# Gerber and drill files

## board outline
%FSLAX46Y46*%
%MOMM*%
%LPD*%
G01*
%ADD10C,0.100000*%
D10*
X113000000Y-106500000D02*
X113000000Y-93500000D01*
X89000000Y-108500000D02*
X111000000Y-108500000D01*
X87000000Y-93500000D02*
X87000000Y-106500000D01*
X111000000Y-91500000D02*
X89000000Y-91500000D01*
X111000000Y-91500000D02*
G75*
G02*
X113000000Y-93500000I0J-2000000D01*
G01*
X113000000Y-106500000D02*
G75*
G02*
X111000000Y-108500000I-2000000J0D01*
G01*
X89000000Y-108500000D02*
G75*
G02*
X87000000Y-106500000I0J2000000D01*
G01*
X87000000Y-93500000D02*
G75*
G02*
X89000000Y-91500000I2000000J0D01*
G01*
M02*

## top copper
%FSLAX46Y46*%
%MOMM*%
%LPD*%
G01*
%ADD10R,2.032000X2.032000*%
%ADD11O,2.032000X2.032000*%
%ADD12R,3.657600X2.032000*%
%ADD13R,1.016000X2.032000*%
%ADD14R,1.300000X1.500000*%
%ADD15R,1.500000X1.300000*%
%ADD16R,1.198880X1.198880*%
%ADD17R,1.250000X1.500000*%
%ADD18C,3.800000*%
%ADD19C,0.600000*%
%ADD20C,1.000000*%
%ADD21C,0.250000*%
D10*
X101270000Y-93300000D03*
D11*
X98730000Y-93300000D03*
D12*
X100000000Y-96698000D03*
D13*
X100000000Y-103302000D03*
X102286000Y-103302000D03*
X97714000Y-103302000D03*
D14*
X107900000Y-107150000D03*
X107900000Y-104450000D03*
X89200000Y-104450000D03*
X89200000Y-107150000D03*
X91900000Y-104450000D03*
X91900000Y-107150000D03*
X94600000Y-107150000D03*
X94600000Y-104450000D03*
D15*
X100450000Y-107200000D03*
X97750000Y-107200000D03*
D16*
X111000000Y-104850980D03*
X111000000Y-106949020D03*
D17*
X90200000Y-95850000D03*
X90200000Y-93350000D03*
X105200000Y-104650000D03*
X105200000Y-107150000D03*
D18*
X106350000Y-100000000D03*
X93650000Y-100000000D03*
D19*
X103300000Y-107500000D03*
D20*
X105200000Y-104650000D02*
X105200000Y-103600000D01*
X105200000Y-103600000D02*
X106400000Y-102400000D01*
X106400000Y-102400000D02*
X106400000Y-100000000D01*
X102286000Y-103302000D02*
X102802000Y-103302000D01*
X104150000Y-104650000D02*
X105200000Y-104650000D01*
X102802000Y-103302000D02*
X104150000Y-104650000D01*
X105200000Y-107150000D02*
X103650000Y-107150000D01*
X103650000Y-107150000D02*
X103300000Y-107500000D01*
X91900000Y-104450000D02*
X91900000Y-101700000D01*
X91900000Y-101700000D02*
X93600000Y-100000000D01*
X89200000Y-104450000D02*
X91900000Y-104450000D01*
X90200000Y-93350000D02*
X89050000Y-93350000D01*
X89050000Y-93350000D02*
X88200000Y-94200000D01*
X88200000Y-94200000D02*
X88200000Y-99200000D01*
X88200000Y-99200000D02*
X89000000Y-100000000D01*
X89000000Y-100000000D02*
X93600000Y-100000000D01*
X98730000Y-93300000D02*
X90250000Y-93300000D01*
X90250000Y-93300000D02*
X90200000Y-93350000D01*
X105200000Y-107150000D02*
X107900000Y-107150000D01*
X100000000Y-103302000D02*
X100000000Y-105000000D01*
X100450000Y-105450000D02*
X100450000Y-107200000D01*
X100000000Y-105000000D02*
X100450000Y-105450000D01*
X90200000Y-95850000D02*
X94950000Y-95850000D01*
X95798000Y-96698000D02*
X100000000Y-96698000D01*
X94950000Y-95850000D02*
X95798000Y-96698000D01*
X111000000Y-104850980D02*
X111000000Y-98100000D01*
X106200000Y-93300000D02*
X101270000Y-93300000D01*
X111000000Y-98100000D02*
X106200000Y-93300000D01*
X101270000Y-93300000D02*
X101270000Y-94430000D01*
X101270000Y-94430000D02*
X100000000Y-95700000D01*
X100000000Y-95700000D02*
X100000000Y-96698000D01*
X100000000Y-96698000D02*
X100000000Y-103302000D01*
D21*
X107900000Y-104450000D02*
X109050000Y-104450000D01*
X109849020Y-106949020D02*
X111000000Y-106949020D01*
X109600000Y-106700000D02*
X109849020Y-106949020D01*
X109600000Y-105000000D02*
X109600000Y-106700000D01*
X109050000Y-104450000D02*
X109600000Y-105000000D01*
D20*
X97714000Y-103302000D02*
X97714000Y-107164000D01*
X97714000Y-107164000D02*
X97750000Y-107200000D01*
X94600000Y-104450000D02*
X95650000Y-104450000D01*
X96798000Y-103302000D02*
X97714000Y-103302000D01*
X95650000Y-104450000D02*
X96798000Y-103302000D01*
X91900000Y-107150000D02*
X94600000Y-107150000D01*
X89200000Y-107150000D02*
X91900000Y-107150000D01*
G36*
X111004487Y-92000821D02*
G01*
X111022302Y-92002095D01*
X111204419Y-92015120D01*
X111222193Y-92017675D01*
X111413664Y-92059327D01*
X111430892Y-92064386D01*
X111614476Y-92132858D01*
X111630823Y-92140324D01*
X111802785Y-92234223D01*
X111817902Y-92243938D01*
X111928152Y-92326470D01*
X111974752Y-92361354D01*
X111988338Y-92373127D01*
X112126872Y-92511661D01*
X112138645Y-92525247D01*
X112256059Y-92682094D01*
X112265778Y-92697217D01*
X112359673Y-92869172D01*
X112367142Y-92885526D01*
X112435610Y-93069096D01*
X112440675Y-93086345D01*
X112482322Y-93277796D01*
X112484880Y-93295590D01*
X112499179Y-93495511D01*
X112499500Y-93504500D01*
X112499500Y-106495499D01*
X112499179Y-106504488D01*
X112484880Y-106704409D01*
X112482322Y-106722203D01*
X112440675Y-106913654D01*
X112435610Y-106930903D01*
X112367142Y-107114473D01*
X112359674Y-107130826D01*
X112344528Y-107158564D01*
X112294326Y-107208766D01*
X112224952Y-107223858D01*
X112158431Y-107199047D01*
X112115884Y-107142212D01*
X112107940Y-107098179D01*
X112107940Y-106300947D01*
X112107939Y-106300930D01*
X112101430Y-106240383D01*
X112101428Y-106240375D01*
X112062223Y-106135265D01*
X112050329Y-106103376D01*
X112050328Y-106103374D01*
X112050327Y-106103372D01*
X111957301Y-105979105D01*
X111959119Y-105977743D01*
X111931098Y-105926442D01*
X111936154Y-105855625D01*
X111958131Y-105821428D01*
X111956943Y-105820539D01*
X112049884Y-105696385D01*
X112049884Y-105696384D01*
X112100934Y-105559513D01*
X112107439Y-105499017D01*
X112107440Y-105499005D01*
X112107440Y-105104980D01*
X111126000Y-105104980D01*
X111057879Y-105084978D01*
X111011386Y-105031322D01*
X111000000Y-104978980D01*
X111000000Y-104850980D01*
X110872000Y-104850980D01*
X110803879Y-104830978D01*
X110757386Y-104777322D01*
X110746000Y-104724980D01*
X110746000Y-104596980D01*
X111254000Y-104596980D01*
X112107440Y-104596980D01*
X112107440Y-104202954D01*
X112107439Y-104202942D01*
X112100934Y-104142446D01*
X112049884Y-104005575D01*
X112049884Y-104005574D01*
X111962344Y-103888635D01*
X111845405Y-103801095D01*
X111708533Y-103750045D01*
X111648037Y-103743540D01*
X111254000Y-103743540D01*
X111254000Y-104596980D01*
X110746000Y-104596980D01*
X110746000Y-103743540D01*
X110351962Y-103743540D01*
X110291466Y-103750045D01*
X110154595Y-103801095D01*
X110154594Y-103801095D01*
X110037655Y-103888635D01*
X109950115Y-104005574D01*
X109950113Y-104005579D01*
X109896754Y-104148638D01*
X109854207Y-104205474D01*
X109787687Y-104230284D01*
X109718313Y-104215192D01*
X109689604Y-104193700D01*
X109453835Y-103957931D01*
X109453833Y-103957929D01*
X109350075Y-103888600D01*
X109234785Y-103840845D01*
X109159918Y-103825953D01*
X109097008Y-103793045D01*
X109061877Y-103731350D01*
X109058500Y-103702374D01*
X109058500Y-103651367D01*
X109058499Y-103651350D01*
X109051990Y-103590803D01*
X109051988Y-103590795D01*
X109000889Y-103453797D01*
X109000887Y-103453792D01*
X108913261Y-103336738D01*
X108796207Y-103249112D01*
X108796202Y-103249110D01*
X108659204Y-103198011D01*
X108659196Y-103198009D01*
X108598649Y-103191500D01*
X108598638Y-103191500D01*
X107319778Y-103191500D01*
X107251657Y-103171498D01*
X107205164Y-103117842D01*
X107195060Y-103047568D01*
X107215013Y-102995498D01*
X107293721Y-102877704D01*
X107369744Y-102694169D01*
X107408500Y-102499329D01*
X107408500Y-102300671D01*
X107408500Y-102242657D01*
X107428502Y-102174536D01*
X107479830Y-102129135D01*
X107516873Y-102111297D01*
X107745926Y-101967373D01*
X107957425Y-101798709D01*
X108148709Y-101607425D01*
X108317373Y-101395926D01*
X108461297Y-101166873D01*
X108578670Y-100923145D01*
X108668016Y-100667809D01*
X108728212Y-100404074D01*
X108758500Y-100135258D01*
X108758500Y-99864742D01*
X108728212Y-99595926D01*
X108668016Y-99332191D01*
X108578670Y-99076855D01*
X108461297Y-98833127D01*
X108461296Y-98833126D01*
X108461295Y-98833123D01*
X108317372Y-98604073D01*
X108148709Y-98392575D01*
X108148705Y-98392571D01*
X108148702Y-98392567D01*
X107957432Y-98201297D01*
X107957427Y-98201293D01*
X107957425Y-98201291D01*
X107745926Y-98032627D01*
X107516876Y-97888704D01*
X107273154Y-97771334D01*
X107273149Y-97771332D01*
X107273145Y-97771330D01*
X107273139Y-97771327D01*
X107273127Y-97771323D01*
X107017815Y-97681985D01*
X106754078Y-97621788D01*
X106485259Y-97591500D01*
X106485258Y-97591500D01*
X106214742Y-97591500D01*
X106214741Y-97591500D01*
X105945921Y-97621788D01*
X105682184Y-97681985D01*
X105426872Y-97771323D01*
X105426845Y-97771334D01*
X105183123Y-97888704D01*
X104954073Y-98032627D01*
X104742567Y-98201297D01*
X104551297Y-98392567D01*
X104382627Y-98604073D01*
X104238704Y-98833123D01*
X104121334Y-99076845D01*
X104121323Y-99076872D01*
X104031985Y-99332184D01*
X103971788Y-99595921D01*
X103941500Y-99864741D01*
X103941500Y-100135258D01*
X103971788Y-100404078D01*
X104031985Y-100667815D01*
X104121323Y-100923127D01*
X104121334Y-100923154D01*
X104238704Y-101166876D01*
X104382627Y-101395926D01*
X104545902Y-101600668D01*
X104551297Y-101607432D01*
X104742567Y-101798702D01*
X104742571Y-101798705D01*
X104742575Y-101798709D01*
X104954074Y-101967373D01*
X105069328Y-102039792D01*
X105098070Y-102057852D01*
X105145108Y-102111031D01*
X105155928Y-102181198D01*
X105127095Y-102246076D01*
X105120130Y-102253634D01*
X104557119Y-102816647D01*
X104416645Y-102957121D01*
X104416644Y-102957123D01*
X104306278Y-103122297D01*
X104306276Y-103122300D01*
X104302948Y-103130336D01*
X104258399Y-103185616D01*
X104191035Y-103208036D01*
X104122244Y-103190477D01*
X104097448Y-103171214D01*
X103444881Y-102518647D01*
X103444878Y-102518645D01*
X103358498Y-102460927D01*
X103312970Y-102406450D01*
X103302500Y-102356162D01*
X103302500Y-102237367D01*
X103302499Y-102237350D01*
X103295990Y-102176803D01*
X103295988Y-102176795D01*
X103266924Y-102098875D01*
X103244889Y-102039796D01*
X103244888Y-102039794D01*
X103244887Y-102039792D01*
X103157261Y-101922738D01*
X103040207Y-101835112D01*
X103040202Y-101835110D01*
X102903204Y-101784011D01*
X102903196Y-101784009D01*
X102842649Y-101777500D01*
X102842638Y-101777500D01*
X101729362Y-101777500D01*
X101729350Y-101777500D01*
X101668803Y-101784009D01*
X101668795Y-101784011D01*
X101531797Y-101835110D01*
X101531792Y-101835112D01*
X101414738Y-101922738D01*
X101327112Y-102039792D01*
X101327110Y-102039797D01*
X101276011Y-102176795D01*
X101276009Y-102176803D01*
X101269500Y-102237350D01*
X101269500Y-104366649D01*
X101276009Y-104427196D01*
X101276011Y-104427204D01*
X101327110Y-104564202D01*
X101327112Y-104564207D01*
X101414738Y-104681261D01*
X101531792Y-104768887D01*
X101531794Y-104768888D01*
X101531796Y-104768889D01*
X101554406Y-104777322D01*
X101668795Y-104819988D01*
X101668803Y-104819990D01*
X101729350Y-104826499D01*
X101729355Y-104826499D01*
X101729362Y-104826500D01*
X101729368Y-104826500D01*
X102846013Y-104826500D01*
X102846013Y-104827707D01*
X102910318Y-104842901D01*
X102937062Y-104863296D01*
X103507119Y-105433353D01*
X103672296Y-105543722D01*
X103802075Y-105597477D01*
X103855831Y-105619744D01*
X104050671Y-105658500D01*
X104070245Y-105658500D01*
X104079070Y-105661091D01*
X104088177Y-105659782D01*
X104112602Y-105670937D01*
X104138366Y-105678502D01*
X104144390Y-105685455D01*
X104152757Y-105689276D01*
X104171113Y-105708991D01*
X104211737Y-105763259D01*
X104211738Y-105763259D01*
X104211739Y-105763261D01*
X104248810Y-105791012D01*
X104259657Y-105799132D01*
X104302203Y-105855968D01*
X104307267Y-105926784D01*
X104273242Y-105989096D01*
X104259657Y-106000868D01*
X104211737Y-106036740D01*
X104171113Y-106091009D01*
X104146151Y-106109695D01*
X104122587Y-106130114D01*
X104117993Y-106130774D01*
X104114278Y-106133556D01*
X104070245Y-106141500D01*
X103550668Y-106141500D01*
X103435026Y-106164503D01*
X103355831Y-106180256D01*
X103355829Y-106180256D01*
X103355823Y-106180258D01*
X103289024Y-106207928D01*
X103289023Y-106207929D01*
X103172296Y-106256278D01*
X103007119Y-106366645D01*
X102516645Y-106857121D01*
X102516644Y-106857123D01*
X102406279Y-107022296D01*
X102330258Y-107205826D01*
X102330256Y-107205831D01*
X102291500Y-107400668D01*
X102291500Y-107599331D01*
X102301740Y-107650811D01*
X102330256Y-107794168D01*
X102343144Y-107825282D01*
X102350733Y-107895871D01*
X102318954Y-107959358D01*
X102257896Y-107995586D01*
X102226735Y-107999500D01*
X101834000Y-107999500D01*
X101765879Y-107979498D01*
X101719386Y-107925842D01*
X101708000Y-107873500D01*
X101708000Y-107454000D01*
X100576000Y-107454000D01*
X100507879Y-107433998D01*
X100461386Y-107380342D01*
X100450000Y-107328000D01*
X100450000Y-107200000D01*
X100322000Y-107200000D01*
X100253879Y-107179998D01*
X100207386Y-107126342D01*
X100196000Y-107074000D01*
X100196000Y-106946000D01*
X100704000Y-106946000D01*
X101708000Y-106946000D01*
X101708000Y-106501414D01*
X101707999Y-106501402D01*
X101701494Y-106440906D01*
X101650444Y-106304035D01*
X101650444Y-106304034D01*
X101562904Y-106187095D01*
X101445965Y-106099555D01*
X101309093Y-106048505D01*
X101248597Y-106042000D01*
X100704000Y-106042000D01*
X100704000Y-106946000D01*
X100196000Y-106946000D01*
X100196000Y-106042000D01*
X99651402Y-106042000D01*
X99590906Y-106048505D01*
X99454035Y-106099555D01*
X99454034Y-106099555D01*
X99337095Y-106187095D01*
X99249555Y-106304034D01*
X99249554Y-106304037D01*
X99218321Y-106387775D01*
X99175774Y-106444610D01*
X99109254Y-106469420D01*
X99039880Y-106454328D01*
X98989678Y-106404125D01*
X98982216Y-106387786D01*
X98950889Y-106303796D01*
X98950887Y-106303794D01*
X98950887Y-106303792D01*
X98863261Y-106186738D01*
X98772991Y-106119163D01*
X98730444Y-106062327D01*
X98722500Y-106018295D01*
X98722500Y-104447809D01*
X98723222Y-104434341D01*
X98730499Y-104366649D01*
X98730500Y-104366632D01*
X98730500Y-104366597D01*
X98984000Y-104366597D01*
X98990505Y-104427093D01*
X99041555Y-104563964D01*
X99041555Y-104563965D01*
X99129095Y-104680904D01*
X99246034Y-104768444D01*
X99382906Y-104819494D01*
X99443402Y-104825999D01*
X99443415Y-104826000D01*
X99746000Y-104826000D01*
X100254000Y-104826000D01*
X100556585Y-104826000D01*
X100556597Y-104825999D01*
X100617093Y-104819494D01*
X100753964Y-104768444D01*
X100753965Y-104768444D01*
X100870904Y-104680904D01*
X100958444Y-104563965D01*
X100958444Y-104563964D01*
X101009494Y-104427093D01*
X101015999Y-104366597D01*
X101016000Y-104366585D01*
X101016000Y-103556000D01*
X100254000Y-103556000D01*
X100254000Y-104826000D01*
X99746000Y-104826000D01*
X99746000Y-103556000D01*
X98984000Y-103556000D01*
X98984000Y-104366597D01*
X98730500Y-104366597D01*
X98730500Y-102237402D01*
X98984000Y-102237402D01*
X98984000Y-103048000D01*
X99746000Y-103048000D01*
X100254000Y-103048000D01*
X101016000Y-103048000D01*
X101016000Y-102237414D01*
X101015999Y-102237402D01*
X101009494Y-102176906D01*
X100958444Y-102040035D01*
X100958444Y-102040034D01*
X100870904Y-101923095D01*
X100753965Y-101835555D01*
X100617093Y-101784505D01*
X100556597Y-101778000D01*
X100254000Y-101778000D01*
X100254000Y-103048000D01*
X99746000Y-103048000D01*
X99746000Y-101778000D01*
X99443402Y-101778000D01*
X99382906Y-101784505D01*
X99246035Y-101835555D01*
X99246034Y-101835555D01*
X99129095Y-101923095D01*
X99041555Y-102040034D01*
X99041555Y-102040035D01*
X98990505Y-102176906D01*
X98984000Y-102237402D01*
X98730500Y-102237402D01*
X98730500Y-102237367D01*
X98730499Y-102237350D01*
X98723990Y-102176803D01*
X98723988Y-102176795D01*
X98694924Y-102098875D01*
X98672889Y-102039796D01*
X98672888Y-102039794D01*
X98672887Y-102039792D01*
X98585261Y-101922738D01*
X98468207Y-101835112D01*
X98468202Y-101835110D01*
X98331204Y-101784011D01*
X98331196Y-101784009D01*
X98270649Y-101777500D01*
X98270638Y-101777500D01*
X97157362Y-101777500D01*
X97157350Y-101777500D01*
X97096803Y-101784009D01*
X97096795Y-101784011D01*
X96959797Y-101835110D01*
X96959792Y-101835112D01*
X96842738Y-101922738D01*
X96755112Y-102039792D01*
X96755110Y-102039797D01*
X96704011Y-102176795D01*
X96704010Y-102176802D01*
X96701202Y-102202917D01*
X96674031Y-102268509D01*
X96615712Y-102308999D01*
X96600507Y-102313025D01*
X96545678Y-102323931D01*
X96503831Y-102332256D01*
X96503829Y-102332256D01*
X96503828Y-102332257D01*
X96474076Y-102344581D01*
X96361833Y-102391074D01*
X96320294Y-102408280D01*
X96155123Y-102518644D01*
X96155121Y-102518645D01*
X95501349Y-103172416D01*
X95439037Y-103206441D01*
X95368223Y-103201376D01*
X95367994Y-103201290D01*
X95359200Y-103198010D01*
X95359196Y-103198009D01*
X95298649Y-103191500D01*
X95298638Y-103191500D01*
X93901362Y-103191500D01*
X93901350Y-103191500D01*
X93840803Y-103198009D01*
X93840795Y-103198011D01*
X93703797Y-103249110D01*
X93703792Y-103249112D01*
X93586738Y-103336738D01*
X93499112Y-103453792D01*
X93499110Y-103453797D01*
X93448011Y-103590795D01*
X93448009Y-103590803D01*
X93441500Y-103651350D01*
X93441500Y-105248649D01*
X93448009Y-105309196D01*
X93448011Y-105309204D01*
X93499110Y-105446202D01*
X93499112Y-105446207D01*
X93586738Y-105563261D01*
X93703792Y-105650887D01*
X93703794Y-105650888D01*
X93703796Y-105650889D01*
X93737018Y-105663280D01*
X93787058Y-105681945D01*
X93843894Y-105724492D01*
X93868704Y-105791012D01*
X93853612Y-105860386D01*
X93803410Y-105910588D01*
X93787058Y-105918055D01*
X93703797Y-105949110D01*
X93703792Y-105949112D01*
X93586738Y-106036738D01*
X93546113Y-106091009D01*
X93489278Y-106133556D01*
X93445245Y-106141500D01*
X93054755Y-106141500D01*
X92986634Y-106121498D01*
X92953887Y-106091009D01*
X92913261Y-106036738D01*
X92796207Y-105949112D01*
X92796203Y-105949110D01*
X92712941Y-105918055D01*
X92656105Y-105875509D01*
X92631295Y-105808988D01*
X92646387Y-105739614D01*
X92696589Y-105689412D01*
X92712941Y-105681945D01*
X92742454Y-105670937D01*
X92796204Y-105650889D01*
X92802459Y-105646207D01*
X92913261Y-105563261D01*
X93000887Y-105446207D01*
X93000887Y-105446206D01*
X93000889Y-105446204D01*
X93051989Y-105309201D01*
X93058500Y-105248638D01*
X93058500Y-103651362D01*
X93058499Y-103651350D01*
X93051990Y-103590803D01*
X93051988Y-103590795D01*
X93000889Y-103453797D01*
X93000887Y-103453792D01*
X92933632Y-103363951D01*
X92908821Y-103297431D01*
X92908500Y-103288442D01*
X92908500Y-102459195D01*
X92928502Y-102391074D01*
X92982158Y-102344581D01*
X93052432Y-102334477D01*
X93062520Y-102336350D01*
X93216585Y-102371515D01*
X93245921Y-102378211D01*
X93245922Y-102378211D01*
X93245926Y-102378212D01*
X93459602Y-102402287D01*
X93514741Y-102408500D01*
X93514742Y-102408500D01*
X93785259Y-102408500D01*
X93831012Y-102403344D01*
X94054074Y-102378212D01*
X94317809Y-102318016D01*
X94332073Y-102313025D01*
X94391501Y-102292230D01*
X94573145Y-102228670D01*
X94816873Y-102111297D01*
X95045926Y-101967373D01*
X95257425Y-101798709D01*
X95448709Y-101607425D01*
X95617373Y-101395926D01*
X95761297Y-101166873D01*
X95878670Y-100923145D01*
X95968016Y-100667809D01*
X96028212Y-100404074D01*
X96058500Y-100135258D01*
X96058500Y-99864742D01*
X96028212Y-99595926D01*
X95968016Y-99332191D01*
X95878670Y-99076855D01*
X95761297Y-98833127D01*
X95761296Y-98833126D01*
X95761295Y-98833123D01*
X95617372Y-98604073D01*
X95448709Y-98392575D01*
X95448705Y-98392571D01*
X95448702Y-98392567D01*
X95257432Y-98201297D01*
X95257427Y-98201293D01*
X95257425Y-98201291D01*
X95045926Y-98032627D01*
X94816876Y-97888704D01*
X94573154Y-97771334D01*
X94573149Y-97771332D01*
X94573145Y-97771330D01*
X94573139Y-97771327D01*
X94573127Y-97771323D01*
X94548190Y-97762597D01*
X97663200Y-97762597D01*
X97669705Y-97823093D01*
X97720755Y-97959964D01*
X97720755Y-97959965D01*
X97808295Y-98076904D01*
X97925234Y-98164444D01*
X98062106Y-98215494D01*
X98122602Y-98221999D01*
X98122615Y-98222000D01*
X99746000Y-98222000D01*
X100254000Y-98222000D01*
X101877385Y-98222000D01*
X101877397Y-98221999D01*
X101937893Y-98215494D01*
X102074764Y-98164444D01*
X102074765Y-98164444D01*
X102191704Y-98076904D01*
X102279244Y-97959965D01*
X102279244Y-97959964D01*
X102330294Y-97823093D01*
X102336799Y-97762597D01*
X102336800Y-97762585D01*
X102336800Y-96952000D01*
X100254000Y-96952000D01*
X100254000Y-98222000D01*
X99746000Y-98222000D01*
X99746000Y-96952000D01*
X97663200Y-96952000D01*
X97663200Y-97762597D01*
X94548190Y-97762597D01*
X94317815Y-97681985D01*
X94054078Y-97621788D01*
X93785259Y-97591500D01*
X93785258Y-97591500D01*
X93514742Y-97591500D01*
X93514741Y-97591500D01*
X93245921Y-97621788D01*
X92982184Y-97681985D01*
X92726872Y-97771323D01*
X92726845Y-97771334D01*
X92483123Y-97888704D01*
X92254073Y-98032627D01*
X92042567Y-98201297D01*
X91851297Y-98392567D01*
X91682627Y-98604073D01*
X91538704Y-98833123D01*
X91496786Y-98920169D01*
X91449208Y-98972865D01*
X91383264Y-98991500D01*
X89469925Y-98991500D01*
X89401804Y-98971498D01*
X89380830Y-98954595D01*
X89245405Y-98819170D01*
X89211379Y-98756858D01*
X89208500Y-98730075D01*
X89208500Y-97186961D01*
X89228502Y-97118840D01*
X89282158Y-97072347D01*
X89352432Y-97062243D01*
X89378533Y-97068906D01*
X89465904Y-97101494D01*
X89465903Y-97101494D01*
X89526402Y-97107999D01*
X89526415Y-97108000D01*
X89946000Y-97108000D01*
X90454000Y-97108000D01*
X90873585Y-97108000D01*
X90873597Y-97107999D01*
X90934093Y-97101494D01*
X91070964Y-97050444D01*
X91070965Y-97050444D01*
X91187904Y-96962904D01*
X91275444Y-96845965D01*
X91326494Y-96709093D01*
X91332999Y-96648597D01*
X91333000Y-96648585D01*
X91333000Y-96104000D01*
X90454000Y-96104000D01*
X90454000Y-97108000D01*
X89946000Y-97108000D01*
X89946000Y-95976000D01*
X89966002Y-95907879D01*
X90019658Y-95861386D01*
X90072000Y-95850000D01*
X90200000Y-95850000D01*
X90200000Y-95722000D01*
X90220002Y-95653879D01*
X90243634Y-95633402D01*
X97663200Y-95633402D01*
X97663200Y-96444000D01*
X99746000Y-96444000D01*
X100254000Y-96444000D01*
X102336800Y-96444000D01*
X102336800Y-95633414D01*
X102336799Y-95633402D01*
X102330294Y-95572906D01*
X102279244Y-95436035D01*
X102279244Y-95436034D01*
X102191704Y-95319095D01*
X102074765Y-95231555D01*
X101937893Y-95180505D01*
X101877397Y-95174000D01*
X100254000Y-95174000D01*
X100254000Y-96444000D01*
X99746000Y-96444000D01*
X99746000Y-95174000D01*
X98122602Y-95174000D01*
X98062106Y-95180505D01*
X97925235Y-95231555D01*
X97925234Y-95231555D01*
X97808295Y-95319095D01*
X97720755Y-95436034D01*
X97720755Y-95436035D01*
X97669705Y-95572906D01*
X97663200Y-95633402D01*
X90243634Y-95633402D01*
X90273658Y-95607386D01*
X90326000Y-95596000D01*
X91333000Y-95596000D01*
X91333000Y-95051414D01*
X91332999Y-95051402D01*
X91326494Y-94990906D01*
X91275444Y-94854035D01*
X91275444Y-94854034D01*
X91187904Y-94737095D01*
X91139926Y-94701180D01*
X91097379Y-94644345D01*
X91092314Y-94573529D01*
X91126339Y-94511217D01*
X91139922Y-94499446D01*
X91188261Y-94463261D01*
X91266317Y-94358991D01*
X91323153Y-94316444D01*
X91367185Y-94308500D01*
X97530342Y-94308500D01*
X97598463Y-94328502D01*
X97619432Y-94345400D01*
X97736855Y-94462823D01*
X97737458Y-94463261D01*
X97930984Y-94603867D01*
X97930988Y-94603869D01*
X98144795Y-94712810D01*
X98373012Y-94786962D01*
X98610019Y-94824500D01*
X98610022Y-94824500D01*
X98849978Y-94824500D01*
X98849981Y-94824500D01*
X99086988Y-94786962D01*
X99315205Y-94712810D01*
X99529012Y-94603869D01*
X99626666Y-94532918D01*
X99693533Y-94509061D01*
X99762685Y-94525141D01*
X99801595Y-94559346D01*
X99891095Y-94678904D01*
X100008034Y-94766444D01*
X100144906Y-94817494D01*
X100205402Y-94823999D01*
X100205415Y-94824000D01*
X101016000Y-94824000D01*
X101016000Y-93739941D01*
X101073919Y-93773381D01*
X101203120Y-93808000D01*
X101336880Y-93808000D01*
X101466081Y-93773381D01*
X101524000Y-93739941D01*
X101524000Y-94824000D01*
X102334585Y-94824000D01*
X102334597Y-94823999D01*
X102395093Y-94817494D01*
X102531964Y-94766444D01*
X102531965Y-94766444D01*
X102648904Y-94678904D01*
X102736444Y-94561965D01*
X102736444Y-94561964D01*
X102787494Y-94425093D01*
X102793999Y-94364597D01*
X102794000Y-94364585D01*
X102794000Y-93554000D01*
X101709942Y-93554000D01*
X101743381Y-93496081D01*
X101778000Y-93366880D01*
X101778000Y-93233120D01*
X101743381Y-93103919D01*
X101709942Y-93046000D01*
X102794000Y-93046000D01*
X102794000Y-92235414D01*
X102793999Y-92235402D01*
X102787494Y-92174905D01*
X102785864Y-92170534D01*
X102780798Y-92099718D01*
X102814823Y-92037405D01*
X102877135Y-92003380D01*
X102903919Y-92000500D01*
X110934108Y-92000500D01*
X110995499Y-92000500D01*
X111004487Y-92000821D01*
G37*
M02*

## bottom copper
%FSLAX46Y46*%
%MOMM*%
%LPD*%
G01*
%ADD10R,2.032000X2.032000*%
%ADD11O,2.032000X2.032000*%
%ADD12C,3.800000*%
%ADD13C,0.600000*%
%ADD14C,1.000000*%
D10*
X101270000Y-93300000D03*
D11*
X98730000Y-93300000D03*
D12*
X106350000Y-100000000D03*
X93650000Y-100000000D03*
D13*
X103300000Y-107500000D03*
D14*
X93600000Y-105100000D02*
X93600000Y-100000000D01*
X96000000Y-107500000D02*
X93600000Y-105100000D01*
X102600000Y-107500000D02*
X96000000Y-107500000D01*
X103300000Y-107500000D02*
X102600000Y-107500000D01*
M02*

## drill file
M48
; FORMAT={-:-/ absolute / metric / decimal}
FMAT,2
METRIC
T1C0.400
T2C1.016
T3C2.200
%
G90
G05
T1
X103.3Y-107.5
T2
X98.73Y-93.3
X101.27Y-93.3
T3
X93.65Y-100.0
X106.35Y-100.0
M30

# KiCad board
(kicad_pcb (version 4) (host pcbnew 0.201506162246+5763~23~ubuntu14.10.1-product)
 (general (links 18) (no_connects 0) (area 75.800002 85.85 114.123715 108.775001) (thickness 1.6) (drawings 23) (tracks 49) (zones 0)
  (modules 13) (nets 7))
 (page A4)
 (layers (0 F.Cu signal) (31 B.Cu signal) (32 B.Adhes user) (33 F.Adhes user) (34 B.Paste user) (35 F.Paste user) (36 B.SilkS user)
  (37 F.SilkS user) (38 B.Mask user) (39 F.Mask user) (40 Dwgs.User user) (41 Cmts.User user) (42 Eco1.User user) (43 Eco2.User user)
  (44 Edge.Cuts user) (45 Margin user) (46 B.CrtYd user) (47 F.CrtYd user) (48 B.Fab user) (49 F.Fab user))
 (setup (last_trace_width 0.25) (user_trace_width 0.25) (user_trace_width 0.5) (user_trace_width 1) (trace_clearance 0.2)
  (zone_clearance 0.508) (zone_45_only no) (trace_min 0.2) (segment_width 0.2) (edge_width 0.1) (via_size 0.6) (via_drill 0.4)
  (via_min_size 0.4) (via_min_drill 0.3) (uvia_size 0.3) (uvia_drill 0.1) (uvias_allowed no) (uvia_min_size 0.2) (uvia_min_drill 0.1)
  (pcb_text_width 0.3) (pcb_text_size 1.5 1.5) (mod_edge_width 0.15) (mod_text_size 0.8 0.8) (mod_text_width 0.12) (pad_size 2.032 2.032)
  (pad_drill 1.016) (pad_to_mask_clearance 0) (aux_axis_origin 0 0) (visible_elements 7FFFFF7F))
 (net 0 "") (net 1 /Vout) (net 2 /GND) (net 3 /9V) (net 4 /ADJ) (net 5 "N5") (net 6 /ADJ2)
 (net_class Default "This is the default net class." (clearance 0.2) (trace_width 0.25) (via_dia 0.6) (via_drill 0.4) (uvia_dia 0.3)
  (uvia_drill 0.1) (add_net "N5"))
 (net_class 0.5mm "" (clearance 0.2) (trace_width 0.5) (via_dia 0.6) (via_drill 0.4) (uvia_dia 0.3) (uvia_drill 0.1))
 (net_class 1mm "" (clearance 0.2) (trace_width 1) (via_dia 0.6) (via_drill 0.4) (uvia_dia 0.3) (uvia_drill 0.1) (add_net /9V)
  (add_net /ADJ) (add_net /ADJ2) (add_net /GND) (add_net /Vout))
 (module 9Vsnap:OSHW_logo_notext (layer B.Cu) (at 100 102.5 180)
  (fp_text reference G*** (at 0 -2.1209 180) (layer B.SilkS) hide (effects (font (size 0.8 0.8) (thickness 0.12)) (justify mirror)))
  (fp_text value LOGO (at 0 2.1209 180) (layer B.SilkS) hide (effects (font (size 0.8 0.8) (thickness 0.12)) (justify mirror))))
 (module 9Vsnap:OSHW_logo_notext (layer F.Cu) (at 110.6 93.8)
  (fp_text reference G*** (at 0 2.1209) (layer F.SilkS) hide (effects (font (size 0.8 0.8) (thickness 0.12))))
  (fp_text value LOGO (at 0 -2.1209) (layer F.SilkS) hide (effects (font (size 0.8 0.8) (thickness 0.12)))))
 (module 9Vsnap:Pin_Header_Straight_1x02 (layer F.Cu) (at 100 93.3 270)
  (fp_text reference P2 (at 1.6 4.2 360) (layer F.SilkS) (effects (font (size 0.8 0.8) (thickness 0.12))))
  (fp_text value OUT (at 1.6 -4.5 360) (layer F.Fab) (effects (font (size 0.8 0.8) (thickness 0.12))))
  (pad 1 thru_hole rect (at 0 -1.27 270) (size 2.032 2.032) (drill 1.016) (layers *.Cu *.Mask F.SilkS) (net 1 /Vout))
  (pad 2 thru_hole oval (at 0 1.27 270) (size 2.032 2.032) (drill 1.016) (layers *.Cu *.Mask F.SilkS) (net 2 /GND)))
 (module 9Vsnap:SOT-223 (layer F.Cu) (at 100 100)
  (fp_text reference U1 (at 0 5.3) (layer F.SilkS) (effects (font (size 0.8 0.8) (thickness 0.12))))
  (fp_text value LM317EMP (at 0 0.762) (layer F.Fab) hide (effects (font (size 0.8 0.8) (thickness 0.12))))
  (pad 2 smd rect (at 0 -3.302) (size 3.6576 2.032) (layers F.Cu F.Paste F.Mask) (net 1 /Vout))
  (pad 2 smd rect (at 0 3.302) (size 1.016 2.032) (layers F.Cu F.Paste F.Mask) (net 1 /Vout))
  (pad 3 smd rect (at 2.286 3.302) (size 1.016 2.032) (layers F.Cu F.Paste F.Mask) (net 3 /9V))
  (pad 1 smd rect (at -2.286 3.302) (size 1.016 2.032) (layers F.Cu F.Paste F.Mask) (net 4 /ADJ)))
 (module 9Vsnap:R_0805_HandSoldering (layer F.Cu) (at 107.9 105.8 90)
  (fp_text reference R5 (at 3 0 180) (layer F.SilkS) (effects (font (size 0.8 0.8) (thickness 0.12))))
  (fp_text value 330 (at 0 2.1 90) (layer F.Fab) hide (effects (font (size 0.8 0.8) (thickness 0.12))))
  (pad 1 smd rect (at -1.35 0 90) (size 1.5 1.3) (layers F.Cu F.Paste F.Mask) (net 2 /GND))
  (pad 2 smd rect (at 1.35 0 90) (size 1.5 1.3) (layers F.Cu F.Paste F.Mask) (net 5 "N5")))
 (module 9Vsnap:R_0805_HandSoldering (layer F.Cu) (at 89.2 105.8 270)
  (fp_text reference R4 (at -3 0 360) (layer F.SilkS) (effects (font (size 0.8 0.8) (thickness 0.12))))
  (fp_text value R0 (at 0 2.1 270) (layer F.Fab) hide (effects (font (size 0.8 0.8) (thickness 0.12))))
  (pad 1 smd rect (at -1.35 0 270) (size 1.5 1.3) (layers F.Cu F.Paste F.Mask) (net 2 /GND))
  (pad 2 smd rect (at 1.35 0 270) (size 1.5 1.3) (layers F.Cu F.Paste F.Mask) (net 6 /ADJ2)))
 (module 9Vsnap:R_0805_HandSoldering (layer F.Cu) (at 91.9 105.8 270)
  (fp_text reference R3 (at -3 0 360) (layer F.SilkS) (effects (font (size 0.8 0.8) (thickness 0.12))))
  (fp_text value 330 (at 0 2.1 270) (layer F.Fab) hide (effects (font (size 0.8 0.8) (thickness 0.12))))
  (pad 1 smd rect (at -1.35 0 270) (size 1.5 1.3) (layers F.Cu F.Paste F.Mask) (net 2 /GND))
  (pad 2 smd rect (at 1.35 0 270) (size 1.5 1.3) (layers F.Cu F.Paste F.Mask) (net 6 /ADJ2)))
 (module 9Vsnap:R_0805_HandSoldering (layer F.Cu) (at 94.6 105.8 90)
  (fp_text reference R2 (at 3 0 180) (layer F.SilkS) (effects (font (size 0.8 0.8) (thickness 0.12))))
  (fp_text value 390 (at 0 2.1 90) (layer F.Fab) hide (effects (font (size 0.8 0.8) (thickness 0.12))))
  (pad 1 smd rect (at -1.35 0 90) (size 1.5 1.3) (layers F.Cu F.Paste F.Mask) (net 6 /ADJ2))
  (pad 2 smd rect (at 1.35 0 90) (size 1.5 1.3) (layers F.Cu F.Paste F.Mask) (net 4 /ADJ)))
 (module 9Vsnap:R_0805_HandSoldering (layer F.Cu) (at 99.1 107.2 180)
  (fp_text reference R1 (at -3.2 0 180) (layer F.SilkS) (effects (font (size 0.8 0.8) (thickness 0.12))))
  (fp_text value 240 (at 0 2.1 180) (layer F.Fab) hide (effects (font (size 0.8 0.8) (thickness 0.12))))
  (pad 1 smd rect (at -1.35 0 180) (size 1.5 1.3) (layers F.Cu F.Paste F.Mask) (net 1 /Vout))
  (pad 2 smd rect (at 1.35 0 180) (size 1.5 1.3) (layers F.Cu F.Paste F.Mask) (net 4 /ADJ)))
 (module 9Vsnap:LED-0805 (layer F.Cu) (at 111 105.9 90)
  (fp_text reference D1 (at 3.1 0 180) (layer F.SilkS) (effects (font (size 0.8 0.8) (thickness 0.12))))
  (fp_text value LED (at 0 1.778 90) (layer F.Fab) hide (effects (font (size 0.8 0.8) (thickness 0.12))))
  (pad 2 smd rect (at 1.04902 0 270) (size 1.19888 1.19888) (layers F.Cu F.Paste F.Mask) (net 1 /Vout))
  (pad 1 smd rect (at -1.04902 0 270) (size 1.19888 1.19888) (layers F.Cu F.Paste F.Mask) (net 5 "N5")))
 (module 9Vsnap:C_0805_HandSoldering (layer F.Cu) (at 90.2 94.6 90)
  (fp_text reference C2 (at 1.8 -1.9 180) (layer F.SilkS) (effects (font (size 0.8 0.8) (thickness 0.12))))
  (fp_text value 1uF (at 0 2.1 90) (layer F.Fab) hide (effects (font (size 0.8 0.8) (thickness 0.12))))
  (pad 1 smd rect (at -1.25 0 90) (size 1.5 1.25) (layers F.Cu F.Paste F.Mask) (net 1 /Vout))
  (pad 2 smd rect (at 1.25 0 90) (size 1.5 1.25) (layers F.Cu F.Paste F.Mask) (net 2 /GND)))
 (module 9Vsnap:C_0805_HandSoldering (layer F.Cu) (at 105.2 105.9 270)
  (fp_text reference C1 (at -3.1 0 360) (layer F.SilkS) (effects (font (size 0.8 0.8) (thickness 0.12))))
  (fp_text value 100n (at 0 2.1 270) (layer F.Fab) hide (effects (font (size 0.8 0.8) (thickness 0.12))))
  (pad 1 smd rect (at -1.25 0 270) (size 1.5 1.25) (layers F.Cu F.Paste F.Mask) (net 3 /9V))
  (pad 2 smd rect (at 1.25 0 270) (size 1.5 1.25) (layers F.Cu F.Paste F.Mask) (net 2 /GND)))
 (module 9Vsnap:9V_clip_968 (layer F.Cu) (at 100 100)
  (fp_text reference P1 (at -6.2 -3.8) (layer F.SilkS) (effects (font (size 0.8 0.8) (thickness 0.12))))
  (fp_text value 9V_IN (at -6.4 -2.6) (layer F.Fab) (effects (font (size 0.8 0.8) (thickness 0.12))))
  (pad 1 thru_hole circle (at 6.35 0) (size 3.8 3.8) (drill 2.2) (layers *.Cu *.Mask F.SilkS) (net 3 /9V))
  (pad 2 thru_hole circle (at -6.35 0) (size 3.8 3.8) (drill 2.2) (layers *.Cu *.Mask F.SilkS) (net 2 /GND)))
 (gr_line (start 113 106.5) (end 113 93.5) (angle 90) (layer Edge.Cuts) (width 0.1))
 (gr_line (start 89 108.5) (end 111 108.5) (angle 90) (layer Edge.Cuts) (width 0.1))
 (gr_line (start 87 93.5) (end 87 106.5) (angle 90) (layer Edge.Cuts) (width 0.1))
 (gr_line (start 111 91.5) (end 89 91.5) (angle 90) (layer Edge.Cuts) (width 0.1))
 (gr_arc (start 111 93.5) (end 111 91.5) (angle 90) (layer Edge.Cuts) (width 0.1))
 (gr_arc (start 111 106.5) (end 113 106.5) (angle 90) (layer Edge.Cuts) (width 0.1))
 (gr_arc (start 89 106.5) (end 89 108.5) (angle 90) (layer Edge.Cuts) (width 0.1))
 (gr_arc (start 89 93.5) (end 87 93.5) (angle 90) (layer Edge.Cuts) (width 0.1))
 (segment (start 105.2 104.65) (end 105.2 103.6) (width 1) (layer F.Cu) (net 3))
 (segment (start 105.2 103.6) (end 106.4 102.4) (width 1) (layer F.Cu) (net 3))
 (segment (start 106.4 102.4) (end 106.4 100) (width 1) (layer F.Cu) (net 3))
 (segment (start 102.286 103.302) (end 102.802 103.302) (width 1) (layer F.Cu) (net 3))
 (segment (start 104.15 104.65) (end 105.2 104.65) (width 1) (layer F.Cu) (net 3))
 (segment (start 102.802 103.302) (end 104.15 104.65) (width 1) (layer F.Cu) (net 3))
 (segment (start 105.2 107.15) (end 103.65 107.15) (width 1) (layer F.Cu) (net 2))
 (segment (start 93.6 105.1) (end 93.6 100) (width 1) (layer B.Cu) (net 2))
 (segment (start 96 107.5) (end 93.6 105.1) (width 1) (layer B.Cu) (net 2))
 (segment (start 102.6 107.5) (end 96 107.5) (width 1) (layer B.Cu) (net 2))
 (segment (start 103.3 107.5) (end 102.6 107.5) (width 1) (layer B.Cu) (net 2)) (via (at 103.3 107.5) (size 0.6) (layers F.Cu B.Cu) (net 2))
 (segment (start 103.65 107.15) (end 103.3 107.5) (width 1) (layer F.Cu) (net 2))
 (segment (start 91.9 104.45) (end 91.9 101.7) (width 1) (layer F.Cu) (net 2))
 (segment (start 91.9 101.7) (end 93.6 100) (width 1) (layer F.Cu) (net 2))
 (segment (start 89.2 104.45) (end 91.9 104.45) (width 1) (layer F.Cu) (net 2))
 (segment (start 90.2 93.35) (end 89.05 93.35) (width 1) (layer F.Cu) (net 2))
 (segment (start 89.05 93.35) (end 88.2 94.2) (width 1) (layer F.Cu) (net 2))
 (segment (start 88.2 94.2) (end 88.2 99.2) (width 1) (layer F.Cu) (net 2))
 (segment (start 88.2 99.2) (end 89 100) (width 1) (layer F.Cu) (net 2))
 (segment (start 89 100) (end 93.6 100) (width 1) (layer F.Cu) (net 2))
 (segment (start 98.73 93.3) (end 90.25 93.3) (width 1) (layer F.Cu) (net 2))
 (segment (start 90.25 93.3) (end 90.2 93.35) (width 1) (layer F.Cu) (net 2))
 (segment (start 105.2 107.15) (end 107.9 107.15) (width 1) (layer F.Cu) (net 2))
 (segment (start 100 103.302) (end 100 105) (width 1) (layer F.Cu) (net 1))
 (segment (start 100.45 105.45) (end 100.45 107.2) (width 1) (layer F.Cu) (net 1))
 (segment (start 100 105) (end 100.45 105.45) (width 1) (layer F.Cu) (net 1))
 (segment (start 90.2 95.85) (end 94.95 95.85) (width 1) (layer F.Cu) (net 1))
 (segment (start 95.798 96.698) (end 100 96.698) (width 1) (layer F.Cu) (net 1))
 (segment (start 94.95 95.85) (end 95.798 96.698) (width 1) (layer F.Cu) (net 1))
 (segment (start 111 104.85098) (end 111 98.1) (width 1) (layer F.Cu) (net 1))
 (segment (start 106.2 93.3) (end 101.27 93.3) (width 1) (layer F.Cu) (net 1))
 (segment (start 111 98.1) (end 106.2 93.3) (width 1) (layer F.Cu) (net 1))
 (segment (start 101.27 93.3) (end 101.27 94.43) (width 1) (layer F.Cu) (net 1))
 (segment (start 101.27 94.43) (end 100 95.7) (width 1) (layer F.Cu) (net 1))
 (segment (start 100 95.7) (end 100 96.698) (width 1) (layer F.Cu) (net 1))
 (segment (start 100 96.698) (end 100 103.302) (width 1) (layer F.Cu) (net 1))
 (segment (start 107.9 104.45) (end 109.05 104.45) (width 0.25) (layer F.Cu) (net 5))
 (segment (start 109.84902 106.94902) (end 111 106.94902) (width 0.25) (layer F.Cu) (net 5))
 (segment (start 109.6 106.7) (end 109.84902 106.94902) (width 0.25) (layer F.Cu) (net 5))
 (segment (start 109.6 105) (end 109.6 106.7) (width 0.25) (layer F.Cu) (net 5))
 (segment (start 109.05 104.45) (end 109.6 105) (width 0.25) (layer F.Cu) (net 5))
 (segment (start 97.714 103.302) (end 97.714 107.164) (width 1) (layer F.Cu) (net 4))
 (segment (start 97.714 107.164) (end 97.75 107.2) (width 1) (layer F.Cu) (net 4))
 (segment (start 94.6 104.45) (end 95.65 104.45) (width 1) (layer F.Cu) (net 4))
 (segment (start 96.798 103.302) (end 97.714 103.302) (width 1) (layer F.Cu) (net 4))
 (segment (start 95.65 104.45) (end 96.798 103.302) (width 1) (layer F.Cu) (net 4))
 (segment (start 91.9 107.15) (end 94.6 107.15) (width 1) (layer F.Cu) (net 6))
 (segment (start 89.2 107.15) (end 91.9 107.15) (width 1) (layer F.Cu) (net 6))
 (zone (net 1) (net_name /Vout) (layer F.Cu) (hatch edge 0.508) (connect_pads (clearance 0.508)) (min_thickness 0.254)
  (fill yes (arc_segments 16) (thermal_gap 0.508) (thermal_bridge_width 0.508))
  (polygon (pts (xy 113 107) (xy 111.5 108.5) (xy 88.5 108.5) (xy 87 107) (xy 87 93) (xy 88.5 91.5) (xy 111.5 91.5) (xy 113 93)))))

